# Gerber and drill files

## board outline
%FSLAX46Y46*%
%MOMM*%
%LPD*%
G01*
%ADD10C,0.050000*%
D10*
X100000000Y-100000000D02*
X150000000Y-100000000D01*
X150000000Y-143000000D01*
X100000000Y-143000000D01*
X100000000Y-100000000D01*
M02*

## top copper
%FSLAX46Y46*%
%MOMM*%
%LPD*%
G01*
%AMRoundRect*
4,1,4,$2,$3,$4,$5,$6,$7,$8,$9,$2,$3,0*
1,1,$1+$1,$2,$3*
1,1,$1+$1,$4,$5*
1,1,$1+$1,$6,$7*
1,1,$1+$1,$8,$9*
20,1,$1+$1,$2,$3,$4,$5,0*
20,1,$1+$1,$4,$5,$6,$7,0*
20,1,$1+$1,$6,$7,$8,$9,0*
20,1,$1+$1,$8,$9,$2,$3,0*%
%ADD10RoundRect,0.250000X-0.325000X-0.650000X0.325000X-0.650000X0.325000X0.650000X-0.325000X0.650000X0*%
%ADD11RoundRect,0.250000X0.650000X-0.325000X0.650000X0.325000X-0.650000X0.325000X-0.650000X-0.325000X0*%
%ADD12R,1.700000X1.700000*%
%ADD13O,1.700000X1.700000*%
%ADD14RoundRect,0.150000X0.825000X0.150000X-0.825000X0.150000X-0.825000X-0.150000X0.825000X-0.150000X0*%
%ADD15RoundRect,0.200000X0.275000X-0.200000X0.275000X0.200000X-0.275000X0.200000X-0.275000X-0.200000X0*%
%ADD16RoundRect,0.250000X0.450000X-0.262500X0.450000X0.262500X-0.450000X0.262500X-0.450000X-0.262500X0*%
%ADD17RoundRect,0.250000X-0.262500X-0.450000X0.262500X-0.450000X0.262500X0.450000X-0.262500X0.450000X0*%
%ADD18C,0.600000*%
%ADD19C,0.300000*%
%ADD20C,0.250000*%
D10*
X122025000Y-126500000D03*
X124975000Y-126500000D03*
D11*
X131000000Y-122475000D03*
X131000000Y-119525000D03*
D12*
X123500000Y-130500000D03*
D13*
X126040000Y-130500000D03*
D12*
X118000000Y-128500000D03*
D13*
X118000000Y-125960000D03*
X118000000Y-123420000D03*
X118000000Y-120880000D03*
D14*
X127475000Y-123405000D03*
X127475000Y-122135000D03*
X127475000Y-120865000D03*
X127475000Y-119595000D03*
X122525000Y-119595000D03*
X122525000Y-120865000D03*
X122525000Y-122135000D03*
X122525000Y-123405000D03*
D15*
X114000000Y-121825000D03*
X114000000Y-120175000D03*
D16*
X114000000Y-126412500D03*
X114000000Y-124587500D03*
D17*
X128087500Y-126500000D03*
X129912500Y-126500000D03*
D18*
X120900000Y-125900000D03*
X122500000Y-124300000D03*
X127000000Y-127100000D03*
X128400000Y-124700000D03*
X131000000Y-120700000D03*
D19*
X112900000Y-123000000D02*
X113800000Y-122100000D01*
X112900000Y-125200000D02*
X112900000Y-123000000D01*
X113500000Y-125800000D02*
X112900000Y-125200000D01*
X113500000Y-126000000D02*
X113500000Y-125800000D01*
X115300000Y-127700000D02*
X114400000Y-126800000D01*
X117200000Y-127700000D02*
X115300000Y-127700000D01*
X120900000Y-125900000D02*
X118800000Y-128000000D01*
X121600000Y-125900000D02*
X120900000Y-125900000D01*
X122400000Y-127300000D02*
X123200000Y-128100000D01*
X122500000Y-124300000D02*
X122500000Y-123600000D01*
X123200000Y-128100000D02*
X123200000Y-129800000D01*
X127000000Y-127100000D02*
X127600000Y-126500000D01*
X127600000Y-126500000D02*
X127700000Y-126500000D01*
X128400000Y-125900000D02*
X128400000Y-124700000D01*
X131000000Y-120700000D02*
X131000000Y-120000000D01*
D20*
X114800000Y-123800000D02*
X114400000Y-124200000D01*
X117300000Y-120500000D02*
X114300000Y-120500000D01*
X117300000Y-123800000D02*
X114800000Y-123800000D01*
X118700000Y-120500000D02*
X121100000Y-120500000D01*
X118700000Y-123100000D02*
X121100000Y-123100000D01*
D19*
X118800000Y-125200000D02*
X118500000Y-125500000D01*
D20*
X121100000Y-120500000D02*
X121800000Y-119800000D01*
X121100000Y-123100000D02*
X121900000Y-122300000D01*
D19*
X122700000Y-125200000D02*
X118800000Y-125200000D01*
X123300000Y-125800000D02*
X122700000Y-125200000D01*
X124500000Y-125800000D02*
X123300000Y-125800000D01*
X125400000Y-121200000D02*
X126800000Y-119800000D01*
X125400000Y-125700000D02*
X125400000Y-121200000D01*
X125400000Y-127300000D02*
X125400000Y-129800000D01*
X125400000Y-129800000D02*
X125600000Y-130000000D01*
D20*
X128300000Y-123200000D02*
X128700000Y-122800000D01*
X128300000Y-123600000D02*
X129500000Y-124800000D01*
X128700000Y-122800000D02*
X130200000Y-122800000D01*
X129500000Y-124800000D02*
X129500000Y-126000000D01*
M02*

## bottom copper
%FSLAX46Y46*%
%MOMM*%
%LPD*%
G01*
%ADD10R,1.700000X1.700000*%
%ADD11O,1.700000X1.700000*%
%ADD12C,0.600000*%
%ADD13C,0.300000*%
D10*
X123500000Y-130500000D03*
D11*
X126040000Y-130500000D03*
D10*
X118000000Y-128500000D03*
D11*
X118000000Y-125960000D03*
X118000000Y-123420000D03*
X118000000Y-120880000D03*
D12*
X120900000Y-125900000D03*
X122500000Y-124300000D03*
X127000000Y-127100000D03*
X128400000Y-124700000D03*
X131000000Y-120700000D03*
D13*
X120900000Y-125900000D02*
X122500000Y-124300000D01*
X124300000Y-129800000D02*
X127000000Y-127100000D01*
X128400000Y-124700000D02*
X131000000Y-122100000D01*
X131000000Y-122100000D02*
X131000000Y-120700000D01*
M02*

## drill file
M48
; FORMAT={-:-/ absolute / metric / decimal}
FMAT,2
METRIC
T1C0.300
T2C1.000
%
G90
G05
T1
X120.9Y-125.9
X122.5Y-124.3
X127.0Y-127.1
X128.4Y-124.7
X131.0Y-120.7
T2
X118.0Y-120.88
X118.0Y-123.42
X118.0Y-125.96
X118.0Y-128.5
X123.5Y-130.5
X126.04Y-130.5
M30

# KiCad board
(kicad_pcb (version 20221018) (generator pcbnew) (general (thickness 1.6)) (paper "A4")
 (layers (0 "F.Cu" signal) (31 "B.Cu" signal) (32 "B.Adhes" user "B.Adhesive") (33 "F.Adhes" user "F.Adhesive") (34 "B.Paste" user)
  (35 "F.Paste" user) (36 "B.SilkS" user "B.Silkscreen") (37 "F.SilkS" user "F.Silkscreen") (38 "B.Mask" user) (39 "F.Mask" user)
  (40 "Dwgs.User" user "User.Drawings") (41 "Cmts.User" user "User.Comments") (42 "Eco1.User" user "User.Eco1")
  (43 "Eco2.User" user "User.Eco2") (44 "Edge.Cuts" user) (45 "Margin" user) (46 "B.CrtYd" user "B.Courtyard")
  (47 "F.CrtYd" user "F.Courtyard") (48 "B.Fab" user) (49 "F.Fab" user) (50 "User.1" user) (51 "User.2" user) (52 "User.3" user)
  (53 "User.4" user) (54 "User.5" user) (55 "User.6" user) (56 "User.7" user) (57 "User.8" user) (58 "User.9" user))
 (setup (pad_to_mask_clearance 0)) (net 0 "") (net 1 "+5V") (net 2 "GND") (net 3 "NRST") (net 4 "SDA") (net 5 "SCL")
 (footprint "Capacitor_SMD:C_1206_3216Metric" (layer "F.Cu") (at 123.5 126.5)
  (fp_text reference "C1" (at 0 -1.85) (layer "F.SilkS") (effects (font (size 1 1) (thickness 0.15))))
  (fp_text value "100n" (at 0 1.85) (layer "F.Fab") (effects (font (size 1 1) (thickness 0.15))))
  (pad "1" smd roundrect (at -1.475 0) (size 1.15 1.8) (layers "F.Cu" "F.Paste" "F.Mask") (roundrect_rratio 0.217391) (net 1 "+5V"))
  (pad "2" smd roundrect (at 1.475 0) (size 1.15 1.8) (layers "F.Cu" "F.Paste" "F.Mask") (roundrect_rratio 0.217391) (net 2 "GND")))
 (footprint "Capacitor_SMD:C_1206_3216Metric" (layer "F.Cu") (at 131 121 90)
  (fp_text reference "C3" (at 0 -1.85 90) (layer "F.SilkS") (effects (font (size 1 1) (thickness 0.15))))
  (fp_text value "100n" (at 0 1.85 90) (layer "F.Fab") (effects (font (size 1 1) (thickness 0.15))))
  (pad "1" smd roundrect (at -1.475 0 90) (size 1.15 1.8) (layers "F.Cu" "F.Paste" "F.Mask") (roundrect_rratio 0.217391) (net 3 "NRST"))
  (pad "2" smd roundrect (at 1.475 0 90) (size 1.15 1.8) (layers "F.Cu" "F.Paste" "F.Mask") (roundrect_rratio 0.217391) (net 1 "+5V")))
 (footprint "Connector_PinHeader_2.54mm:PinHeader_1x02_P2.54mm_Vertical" (layer "F.Cu") (at 123.5 130.5 90)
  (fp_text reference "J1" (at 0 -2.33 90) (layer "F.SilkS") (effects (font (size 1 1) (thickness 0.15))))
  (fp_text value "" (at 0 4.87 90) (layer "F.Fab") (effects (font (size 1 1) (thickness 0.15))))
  (pad "1" thru_hole rect (at 0 0 90) (size 1.7 1.7) (drill 1) (layers "*.Cu" "*.Mask") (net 1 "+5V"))
  (pad "2" thru_hole oval (at 0 2.54 90) (size 1.7 1.7) (drill 1) (layers "*.Cu" "*.Mask") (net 2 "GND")))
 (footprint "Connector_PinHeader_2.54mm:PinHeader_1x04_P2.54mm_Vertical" (layer "F.Cu") (at 118 128.5 180)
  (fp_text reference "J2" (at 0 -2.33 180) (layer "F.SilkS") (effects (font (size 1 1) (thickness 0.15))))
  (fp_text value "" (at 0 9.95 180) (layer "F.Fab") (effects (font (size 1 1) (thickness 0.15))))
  (pad "1" thru_hole rect (at 0 0 180) (size 1.7 1.7) (drill 1) (layers "*.Cu" "*.Mask") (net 1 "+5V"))
  (pad "2" thru_hole oval (at 0 2.54 180) (size 1.7 1.7) (drill 1) (layers "*.Cu" "*.Mask") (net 2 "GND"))
  (pad "3" thru_hole oval (at 0 5.08 180) (size 1.7 1.7) (drill 1) (layers "*.Cu" "*.Mask") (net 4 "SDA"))
  (pad "4" thru_hole oval (at 0 7.62 180) (size 1.7 1.7) (drill 1) (layers "*.Cu" "*.Mask") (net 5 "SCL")))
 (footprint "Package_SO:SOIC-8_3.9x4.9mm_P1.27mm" (layer "F.Cu") (at 125 121.5 180)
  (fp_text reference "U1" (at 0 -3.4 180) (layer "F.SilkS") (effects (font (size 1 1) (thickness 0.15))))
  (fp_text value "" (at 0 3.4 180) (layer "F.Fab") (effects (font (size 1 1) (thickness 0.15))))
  (pad "1" smd roundrect (at -2.475 -1.905 180) (size 1.95 0.6) (layers "F.Cu" "F.Paste" "F.Mask") (roundrect_rratio 0.25) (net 3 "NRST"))
  (pad "2" smd roundrect (at -2.475 -0.635 180) (size 1.95 0.6) (layers "F.Cu" "F.Paste" "F.Mask") (roundrect_rratio 0.25))
  (pad "3" smd roundrect (at -2.475 0.635 180) (size 1.95 0.6) (layers "F.Cu" "F.Paste" "F.Mask") (roundrect_rratio 0.25))
  (pad "4" smd roundrect (at -2.475 1.905 180) (size 1.95 0.6) (layers "F.Cu" "F.Paste" "F.Mask") (roundrect_rratio 0.25) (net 2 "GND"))
  (pad "5" smd roundrect (at 2.475 1.905 180) (size 1.95 0.6) (layers "F.Cu" "F.Paste" "F.Mask") (roundrect_rratio 0.25) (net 5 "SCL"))
  (pad "6" smd roundrect (at 2.475 0.635 180) (size 1.95 0.6) (layers "F.Cu" "F.Paste" "F.Mask") (roundrect_rratio 0.25))
  (pad "7" smd roundrect (at 2.475 -0.635 180) (size 1.95 0.6) (layers "F.Cu" "F.Paste" "F.Mask") (roundrect_rratio 0.25) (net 4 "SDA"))
  (pad "8" smd roundrect (at 2.475 -1.905 180) (size 1.95 0.6) (layers "F.Cu" "F.Paste" "F.Mask") (roundrect_rratio 0.25) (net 1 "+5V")))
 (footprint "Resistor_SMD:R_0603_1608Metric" (layer "F.Cu") (at 114 121 90)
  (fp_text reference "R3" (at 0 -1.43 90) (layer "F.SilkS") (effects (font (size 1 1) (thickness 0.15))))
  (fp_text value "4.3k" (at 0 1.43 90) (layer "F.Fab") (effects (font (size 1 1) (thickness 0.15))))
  (pad "1" smd roundrect (at -0.825 0 90) (size 0.8 0.95) (layers "F.Cu" "F.Paste" "F.Mask") (roundrect_rratio 0.25) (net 1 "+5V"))
  (pad "2" smd roundrect (at 0.825 0 90) (size 0.8 0.95) (layers "F.Cu" "F.Paste" "F.Mask") (roundrect_rratio 0.25) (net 5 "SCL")))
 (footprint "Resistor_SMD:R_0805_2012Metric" (layer "F.Cu") (at 114 125.5 90)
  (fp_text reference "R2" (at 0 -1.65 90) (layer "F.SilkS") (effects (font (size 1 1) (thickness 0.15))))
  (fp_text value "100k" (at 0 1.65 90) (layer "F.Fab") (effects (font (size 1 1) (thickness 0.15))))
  (pad "1" smd roundrect (at -0.9125 0 90) (size 1.025 1.4) (layers "F.Cu" "F.Paste" "F.Mask") (roundrect_rratio 0.243902) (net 1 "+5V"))
  (pad "2" smd roundrect (at 0.9125 0 90) (size 1.025 1.4) (layers "F.Cu" "F.Paste" "F.Mask") (roundrect_rratio 0.243902) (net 4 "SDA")))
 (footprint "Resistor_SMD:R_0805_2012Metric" (layer "F.Cu") (at 129 126.5)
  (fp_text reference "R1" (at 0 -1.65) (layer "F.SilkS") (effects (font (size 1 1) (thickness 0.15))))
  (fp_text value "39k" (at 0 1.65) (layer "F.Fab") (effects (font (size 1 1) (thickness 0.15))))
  (pad "1" smd roundrect (at -0.9125 0) (size 1.025 1.4) (layers "F.Cu" "F.Paste" "F.Mask") (roundrect_rratio 0.243902) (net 1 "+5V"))
  (pad "2" smd roundrect (at 0.9125 0) (size 1.025 1.4) (layers "F.Cu" "F.Paste" "F.Mask") (roundrect_rratio 0.243902) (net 3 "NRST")))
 (gr_rect (start 100 100) (end 150 143) (stroke (width 0.05) (type default)) (fill none) (layer "Edge.Cuts"))
 (segment (start 112.9 123) (end 113.8 122.1) (width 0.3) (layer "F.Cu") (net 1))
 (segment (start 112.9 125.2) (end 112.9 123) (width 0.3) (layer "F.Cu") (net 1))
 (segment (start 113.5 125.8) (end 112.9 125.2) (width 0.3) (layer "F.Cu") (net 1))
 (segment (start 113.5 126) (end 113.5 125.8) (width 0.3) (layer "F.Cu") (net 1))
 (segment (start 115.3 127.7) (end 114.4 126.8) (width 0.3) (layer "F.Cu") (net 1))
 (segment (start 117.2 127.7) (end 115.3 127.7) (width 0.3) (layer "F.Cu") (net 1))
 (segment (start 120.9 125.9) (end 118.8 128) (width 0.3) (layer "F.Cu") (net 1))
 (segment (start 121.6 125.9) (end 120.9 125.9) (width 0.3) (layer "F.Cu") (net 1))
 (segment (start 122.4 127.3) (end 123.2 128.1) (width 0.3) (layer "F.Cu") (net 1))
 (segment (start 122.5 124.3) (end 122.5 123.6) (width 0.3) (layer "F.Cu") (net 1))
 (segment (start 123.2 128.1) (end 123.2 129.8) (width 0.3) (layer "F.Cu") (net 1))
 (segment (start 127 127.1) (end 127.6 126.5) (width 0.3) (layer "F.Cu") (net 1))
 (segment (start 127.6 126.5) (end 127.7 126.5) (width 0.3) (layer "F.Cu") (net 1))
 (segment (start 128.4 125.9) (end 128.4 124.7) (width 0.3) (layer "F.Cu") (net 1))
 (segment (start 131 120.7) (end 131 120) (width 0.3) (layer "F.Cu") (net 1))
 (via (at 120.9 125.9) (size 0.6) (drill 0.3) (layers "F.Cu" "B.Cu") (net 1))
 (via (at 122.5 124.3) (size 0.6) (drill 0.3) (layers "F.Cu" "B.Cu") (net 1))
 (via (at 127 127.1) (size 0.6) (drill 0.3) (layers "F.Cu" "B.Cu") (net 1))
 (via (at 128.4 124.7) (size 0.6) (drill 0.3) (layers "F.Cu" "B.Cu") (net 1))
 (via (at 131 120.7) (size 0.6) (drill 0.3) (layers "F.Cu" "B.Cu") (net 1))
 (segment (start 114.8 123.8) (end 114.4 124.2) (width 0.25) (layer "F.Cu") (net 4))
 (segment (start 117.3 120.5) (end 114.3 120.5) (width 0.25) (layer "F.Cu") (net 5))
 (segment (start 117.3 123.8) (end 114.8 123.8) (width 0.25) (layer "F.Cu") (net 4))
 (segment (start 118.7 120.5) (end 121.1 120.5) (width 0.25) (layer "F.Cu") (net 5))
 (segment (start 118.7 123.1) (end 121.1 123.1) (width 0.25) (layer "F.Cu") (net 4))
 (segment (start 118.8 125.2) (end 118.5 125.5) (width 0.3) (layer "F.Cu") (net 2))
 (segment (start 120.9 125.9) (end 122.5 124.3) (width 0.3) (layer "B.Cu") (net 1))
 (segment (start 121.1 120.5) (end 121.8 119.8) (width 0.25) (layer "F.Cu") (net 5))
 (segment (start 121.1 123.1) (end 121.9 122.3) (width 0.25) (layer "F.Cu") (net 4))
 (segment (start 122.7 125.2) (end 118.8 125.2) (width 0.3) (layer "F.Cu") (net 2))
 (segment (start 123.3 125.8) (end 122.7 125.2) (width 0.3) (layer "F.Cu") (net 2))
 (segment (start 124.3 129.8) (end 127 127.1) (width 0.3) (layer "B.Cu") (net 1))
 (segment (start 124.5 125.8) (end 123.3 125.8) (width 0.3) (layer "F.Cu") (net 2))
 (segment (start 125.4 121.2) (end 126.8 119.8) (width 0.3) (layer "F.Cu") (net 2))
 (segment (start 125.4 125.7) (end 125.4 121.2) (width 0.3) (layer "F.Cu") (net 2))
 (segment (start 125.4 127.3) (end 125.4 129.8) (width 0.3) (layer "F.Cu") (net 2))
 (segment (start 125.4 129.8) (end 125.6 130) (width 0.3) (layer "F.Cu") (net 2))
 (segment (start 128.3 123.2) (end 128.7 122.8) (width 0.25) (layer "F.Cu") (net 3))
 (segment (start 128.3 123.6) (end 129.5 124.8) (width 0.25) (layer "F.Cu") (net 3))
 (segment (start 128.4 124.7) (end 131 122.1) (width 0.3) (layer "B.Cu") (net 1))
 (segment (start 128.7 122.8) (end 130.2 122.8) (width 0.25) (layer "F.Cu") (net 3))
 (segment (start 129.5 124.8) (end 129.5 126) (width 0.25) (layer "F.Cu") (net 3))
 (segment (start 131 122.1) (end 131 120.7) (width 0.3) (layer "B.Cu") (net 1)))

